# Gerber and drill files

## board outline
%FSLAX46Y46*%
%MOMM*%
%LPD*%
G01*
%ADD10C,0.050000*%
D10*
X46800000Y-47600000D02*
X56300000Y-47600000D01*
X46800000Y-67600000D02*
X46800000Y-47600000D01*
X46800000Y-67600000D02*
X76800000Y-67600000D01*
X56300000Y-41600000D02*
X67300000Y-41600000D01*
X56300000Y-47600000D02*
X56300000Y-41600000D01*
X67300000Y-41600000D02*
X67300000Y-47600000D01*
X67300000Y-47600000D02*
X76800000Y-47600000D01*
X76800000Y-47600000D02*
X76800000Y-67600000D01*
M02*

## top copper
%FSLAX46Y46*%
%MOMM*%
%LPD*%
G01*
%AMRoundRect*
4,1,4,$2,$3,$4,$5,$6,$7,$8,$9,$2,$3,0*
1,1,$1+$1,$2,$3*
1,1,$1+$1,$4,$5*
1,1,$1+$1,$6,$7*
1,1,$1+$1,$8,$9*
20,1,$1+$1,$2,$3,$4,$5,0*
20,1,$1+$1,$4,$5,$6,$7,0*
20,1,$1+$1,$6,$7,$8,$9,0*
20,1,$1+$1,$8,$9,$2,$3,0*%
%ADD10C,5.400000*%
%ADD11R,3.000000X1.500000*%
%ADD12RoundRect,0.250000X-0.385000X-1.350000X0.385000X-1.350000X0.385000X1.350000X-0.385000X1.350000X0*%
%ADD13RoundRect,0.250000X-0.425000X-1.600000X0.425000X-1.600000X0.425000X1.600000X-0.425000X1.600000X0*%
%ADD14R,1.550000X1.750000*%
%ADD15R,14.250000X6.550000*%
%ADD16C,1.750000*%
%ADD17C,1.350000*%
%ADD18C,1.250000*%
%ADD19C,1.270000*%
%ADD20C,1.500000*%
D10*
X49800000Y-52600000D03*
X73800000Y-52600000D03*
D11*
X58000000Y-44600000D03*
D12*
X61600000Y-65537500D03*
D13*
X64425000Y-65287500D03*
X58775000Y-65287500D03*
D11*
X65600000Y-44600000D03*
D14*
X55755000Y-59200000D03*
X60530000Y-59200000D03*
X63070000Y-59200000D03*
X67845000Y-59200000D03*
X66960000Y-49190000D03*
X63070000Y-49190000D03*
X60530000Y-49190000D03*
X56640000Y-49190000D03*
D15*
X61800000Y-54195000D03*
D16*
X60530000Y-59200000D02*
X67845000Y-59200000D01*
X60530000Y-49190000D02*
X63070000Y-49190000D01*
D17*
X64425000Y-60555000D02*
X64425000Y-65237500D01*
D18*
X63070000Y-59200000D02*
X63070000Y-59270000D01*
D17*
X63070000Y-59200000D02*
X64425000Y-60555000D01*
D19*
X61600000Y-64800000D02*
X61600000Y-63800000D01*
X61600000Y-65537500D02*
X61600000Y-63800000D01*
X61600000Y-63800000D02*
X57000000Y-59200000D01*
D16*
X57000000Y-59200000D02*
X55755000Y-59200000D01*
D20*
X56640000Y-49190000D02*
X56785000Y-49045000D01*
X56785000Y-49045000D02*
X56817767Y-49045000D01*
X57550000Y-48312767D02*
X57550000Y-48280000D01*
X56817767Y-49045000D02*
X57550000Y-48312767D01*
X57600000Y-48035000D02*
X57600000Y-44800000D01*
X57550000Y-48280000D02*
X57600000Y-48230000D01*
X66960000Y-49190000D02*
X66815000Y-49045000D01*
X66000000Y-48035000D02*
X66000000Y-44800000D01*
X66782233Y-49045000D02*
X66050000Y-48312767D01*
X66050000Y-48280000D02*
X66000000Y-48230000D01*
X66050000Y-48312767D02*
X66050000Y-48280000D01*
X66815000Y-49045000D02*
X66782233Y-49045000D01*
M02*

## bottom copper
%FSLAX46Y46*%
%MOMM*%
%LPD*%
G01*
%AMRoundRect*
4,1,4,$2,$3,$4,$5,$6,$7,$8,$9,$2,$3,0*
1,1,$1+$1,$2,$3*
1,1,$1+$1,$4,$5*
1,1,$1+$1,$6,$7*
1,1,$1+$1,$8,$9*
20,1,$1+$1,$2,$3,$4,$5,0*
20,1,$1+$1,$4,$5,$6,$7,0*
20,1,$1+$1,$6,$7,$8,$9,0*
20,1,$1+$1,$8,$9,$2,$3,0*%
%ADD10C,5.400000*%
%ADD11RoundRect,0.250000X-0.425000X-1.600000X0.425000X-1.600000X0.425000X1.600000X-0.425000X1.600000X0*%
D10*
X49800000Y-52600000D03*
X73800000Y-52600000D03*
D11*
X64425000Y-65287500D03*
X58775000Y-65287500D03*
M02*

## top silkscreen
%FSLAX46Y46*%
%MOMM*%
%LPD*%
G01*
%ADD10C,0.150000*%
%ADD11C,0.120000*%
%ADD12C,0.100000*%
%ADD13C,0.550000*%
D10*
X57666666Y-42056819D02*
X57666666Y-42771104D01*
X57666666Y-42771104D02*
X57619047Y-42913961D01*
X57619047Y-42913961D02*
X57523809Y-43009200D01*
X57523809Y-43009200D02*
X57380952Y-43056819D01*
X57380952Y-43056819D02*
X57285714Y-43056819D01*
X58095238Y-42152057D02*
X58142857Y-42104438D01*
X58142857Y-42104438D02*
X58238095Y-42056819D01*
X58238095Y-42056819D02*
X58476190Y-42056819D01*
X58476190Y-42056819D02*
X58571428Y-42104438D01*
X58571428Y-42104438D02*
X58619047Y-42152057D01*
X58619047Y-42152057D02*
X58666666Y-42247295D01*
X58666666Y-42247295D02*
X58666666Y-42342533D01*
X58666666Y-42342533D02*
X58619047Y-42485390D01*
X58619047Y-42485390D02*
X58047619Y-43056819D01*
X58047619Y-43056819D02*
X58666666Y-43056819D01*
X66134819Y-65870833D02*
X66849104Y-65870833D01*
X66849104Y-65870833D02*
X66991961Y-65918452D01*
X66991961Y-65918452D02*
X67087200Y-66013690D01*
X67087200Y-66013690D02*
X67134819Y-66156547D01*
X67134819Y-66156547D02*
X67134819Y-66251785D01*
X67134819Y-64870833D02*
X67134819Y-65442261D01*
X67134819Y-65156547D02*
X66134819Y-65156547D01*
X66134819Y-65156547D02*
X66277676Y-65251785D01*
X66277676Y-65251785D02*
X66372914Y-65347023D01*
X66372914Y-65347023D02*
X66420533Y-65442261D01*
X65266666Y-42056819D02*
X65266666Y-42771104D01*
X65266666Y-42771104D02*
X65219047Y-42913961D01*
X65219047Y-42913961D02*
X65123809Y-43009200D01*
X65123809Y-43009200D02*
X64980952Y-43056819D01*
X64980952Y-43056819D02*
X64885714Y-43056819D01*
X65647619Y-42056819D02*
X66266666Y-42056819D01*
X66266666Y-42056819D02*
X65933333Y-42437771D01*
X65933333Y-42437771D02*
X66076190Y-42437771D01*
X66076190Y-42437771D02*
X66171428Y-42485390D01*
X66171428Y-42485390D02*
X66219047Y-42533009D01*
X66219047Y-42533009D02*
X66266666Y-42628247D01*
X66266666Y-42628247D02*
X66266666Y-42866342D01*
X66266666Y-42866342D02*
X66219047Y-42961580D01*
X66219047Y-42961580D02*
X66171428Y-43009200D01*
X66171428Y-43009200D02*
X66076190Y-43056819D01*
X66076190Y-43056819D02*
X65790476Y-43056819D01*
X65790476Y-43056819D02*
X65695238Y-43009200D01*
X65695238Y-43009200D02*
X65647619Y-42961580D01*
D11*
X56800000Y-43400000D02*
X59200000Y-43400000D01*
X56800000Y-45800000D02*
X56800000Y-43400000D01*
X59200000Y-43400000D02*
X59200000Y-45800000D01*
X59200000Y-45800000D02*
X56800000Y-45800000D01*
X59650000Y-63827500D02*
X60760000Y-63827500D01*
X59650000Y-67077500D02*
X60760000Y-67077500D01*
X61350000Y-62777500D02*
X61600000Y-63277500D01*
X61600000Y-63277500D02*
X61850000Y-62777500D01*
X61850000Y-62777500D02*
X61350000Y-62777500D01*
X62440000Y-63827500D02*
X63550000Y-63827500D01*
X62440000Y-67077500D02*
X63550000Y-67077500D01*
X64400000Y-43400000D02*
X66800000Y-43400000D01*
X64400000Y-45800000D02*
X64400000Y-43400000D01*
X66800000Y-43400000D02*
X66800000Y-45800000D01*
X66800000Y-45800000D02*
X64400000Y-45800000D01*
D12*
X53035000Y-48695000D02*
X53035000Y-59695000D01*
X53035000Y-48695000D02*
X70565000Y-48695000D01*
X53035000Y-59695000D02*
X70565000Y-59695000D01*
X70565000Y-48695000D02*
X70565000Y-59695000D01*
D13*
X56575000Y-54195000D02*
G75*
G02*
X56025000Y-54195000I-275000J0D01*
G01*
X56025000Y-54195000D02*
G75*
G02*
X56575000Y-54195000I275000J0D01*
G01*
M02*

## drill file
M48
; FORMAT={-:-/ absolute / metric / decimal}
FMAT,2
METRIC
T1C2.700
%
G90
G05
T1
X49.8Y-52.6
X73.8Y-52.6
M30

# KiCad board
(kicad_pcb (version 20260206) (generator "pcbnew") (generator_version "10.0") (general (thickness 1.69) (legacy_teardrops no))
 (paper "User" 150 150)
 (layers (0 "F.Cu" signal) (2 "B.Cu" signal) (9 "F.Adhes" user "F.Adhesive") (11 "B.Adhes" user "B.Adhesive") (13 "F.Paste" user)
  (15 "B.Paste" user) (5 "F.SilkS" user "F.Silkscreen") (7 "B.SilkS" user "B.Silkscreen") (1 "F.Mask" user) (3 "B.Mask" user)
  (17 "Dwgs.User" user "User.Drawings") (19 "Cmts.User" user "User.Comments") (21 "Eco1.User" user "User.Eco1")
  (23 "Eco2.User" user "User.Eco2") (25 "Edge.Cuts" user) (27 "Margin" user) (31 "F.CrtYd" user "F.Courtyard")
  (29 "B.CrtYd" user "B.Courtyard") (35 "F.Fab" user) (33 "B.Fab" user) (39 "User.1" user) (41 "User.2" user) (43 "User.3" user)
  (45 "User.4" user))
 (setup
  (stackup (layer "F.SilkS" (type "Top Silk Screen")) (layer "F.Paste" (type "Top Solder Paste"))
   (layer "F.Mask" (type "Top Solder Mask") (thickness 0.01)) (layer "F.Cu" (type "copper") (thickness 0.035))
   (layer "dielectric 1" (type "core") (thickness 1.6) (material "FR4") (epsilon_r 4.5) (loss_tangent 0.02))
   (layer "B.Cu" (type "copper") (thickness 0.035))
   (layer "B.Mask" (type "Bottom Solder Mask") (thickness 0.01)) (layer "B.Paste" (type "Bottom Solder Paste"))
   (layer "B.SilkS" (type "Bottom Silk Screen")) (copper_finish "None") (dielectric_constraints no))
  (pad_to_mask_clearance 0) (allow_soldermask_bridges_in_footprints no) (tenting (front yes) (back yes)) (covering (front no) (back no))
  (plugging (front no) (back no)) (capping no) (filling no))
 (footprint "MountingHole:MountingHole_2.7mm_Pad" (layer "F.Cu") (at 49.8 52.6)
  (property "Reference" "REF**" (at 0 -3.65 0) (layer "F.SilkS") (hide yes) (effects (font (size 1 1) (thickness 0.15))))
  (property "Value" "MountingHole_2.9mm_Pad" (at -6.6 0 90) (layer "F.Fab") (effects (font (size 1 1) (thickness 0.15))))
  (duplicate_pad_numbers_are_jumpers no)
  (pad "1" thru_hole circle (at 0 0) (size 5.4 5.4) (drill 2.7) (layers "*.Cu" "*.Mask") (remove_unused_layers no) (zone_connect 2)))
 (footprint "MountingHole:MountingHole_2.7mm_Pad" (layer "F.Cu") (at 73.8 52.6)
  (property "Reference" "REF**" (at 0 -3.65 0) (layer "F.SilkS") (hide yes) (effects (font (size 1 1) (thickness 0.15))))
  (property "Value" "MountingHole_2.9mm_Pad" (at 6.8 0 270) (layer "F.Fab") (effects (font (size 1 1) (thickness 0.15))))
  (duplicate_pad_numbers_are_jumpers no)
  (pad "1" thru_hole circle (at 0 0) (size 5.4 5.4) (drill 2.7) (layers "*.Cu" "*.Mask") (remove_unused_layers no) (zone_connect 2)))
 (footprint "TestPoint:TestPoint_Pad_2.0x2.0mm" (layer "F.Cu") (at 58 44.6)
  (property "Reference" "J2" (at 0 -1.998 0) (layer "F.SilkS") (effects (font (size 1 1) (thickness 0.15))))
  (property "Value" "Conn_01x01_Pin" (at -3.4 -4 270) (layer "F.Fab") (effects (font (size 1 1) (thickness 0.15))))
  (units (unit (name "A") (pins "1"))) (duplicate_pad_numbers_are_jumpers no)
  (fp_line (start -1.2 -1.2) (end 1.2 -1.2) (stroke (width 0.12) (type solid)) (layer "F.SilkS"))
  (fp_line (start -1.2 1.2) (end -1.2 -1.2) (stroke (width 0.12) (type solid)) (layer "F.SilkS"))
  (fp_line (start 1.2 -1.2) (end 1.2 1.2) (stroke (width 0.12) (type solid)) (layer "F.SilkS"))
  (fp_line (start 1.2 1.2) (end -1.2 1.2) (stroke (width 0.12) (type solid)) (layer "F.SilkS"))
  (pad "1" smd rect (at 0 0) (size 3 1.5) (layers "F.Cu" "F.Mask") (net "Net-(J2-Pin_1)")))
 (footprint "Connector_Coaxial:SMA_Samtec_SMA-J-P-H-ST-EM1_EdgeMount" (layer "F.Cu") (at 61.6 65.5375 -90)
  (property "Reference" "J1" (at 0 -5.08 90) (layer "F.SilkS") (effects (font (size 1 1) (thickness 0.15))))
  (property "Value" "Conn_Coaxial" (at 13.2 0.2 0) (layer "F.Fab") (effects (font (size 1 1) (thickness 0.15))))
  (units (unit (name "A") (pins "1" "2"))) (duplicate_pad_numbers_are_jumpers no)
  (fp_line (start -1.71 1.95) (end -1.71 0.84) (stroke (width 0.12) (type solid)) (layer "F.SilkS"))
  (fp_line (start 1.54 1.95) (end 1.54 0.84) (stroke (width 0.12) (type solid)) (layer "F.SilkS"))
  (fp_line (start -2.76 0.25) (end -2.26 0) (stroke (width 0.12) (type solid)) (layer "F.SilkS"))
  (fp_line (start -2.26 0) (end -2.76 -0.25) (stroke (width 0.12) (type solid)) (layer "F.SilkS"))
  (fp_line (start -2.76 -0.25) (end -2.76 0.25) (stroke (width 0.12) (type solid)) (layer "F.SilkS"))
  (fp_line (start -1.71 -0.84) (end -1.71 -1.95) (stroke (width 0.12) (type solid)) (layer "F.SilkS"))
  (fp_line (start 1.54 -0.84) (end 1.54 -1.95) (stroke (width 0.12) (type solid)) (layer "F.SilkS"))
  (pad "1" smd roundrect (at 0 0) (size 1.27 3.2) (layers "F.Cu" "F.Mask") (roundrect_rratio 0.1968503937) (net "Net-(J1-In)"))
  (pad "2" smd roundrect (at -0.25 -2.825) (size 1.35 3.7) (layers "F.Cu" "F.Mask") (roundrect_rratio 0.1851851852) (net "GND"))
  (pad "2" smd roundrect (at -0.25 -2.825) (size 1.35 3.7) (layers "B.Cu" "B.Mask") (roundrect_rratio 0.1851851852) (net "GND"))
  (pad "2" smd roundrect (at -0.25 2.825) (size 1.35 3.7) (layers "F.Cu" "F.Mask") (roundrect_rratio 0.1851851852) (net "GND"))
  (pad "2" smd roundrect (at -0.25 2.825) (size 1.35 3.7) (layers "B.Cu" "B.Mask") (roundrect_rratio 0.1851851852) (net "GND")))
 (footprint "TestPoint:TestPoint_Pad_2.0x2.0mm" (layer "F.Cu") (at 65.6 44.6)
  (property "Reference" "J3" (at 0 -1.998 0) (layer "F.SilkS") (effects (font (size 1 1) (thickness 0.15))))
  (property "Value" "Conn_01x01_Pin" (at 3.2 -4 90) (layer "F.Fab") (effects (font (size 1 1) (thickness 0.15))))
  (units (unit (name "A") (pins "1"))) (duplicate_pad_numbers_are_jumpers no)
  (fp_line (start -1.2 -1.2) (end 1.2 -1.2) (stroke (width 0.12) (type solid)) (layer "F.SilkS"))
  (fp_line (start -1.2 1.2) (end -1.2 -1.2) (stroke (width 0.12) (type solid)) (layer "F.SilkS"))
  (fp_line (start 1.2 -1.2) (end 1.2 1.2) (stroke (width 0.12) (type solid)) (layer "F.SilkS"))
  (fp_line (start 1.2 1.2) (end -1.2 1.2) (stroke (width 0.12) (type solid)) (layer "F.SilkS"))
  (pad "1" smd rect (at 0 0) (size 3 1.5) (layers "F.Cu" "F.Mask") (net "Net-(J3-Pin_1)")))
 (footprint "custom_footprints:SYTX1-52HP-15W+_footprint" (layer "F.Cu") (at 61.8 54.195)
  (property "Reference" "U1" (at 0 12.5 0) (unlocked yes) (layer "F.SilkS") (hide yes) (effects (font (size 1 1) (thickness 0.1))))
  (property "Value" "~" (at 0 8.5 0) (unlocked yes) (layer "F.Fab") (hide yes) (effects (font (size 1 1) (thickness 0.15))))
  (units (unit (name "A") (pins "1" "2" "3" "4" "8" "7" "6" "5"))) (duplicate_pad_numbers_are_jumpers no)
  (fp_line (start -8.765 -5.5) (end -8.765 5.5) (stroke (width 0.1) (type solid)) (layer "F.SilkS"))
  (fp_line (start -8.765 -5.5) (end 8.765 -5.5) (stroke (width 0.1) (type solid)) (layer "F.SilkS"))
  (fp_line (start -8.765 5.5) (end 8.765 5.5) (stroke (width 0.1) (type solid)) (layer "F.SilkS"))
  (fp_line (start 8.765 -5.5) (end 8.765 5.5) (stroke (width 0.1) (type solid)) (layer "F.SilkS"))
  (fp_circle (center -5.5 0) (end -6 0) (stroke (width 0.1) (type solid)) (fill yes) (layer "F.SilkS"))
  (pad "1" smd rect (at -6.045 5.005) (size 1.55 1.75) (layers "F.Cu" "F.Mask" "F.Paste") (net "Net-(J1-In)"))
  (pad "2" smd rect (at -1.27 5.005) (size 1.55 1.75) (layers "F.Cu" "F.Mask" "F.Paste") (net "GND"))
  (pad "3" smd rect (at 1.27 5.005) (size 1.55 1.75) (layers "F.Cu" "F.Mask" "F.Paste") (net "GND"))
  (pad "4" smd rect (at 6.045 5.005) (size 1.55 1.75) (layers "F.Cu" "F.Mask" "F.Paste") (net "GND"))
  (pad "5" smd rect (at 5.16 -5.005) (size 1.55 1.75) (layers "F.Cu" "F.Mask" "F.Paste") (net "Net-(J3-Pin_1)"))
  (pad "6" smd rect (at 1.27 -5.005) (size 1.55 1.75) (layers "F.Cu" "F.Mask" "F.Paste") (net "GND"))
  (pad "7" smd rect (at -1.27 -5.005) (size 1.55 1.75) (layers "F.Cu" "F.Mask" "F.Paste") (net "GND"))
  (pad "8" smd rect (at -5.16 -5.005) (size 1.55 1.75) (layers "F.Cu" "F.Mask" "F.Paste") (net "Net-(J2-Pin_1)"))
  (pad "9" smd rect (at 0 0) (size 14.25 6.55) (layers "F.Cu" "F.Mask" "F.Paste")))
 (gr_line (start 46.8 47.6) (end 56.3 47.6) (stroke (width 0.05) (type solid)) (layer "Edge.Cuts"))
 (gr_line (start 46.8 67.6) (end 46.8 47.6) (stroke (width 0.05) (type solid)) (layer "Edge.Cuts"))
 (gr_line (start 46.8 67.6) (end 76.8 67.6) (stroke (width 0.05) (type solid)) (layer "Edge.Cuts"))
 (gr_line (start 56.3 41.6) (end 67.3 41.6) (stroke (width 0.05) (type solid)) (layer "Edge.Cuts"))
 (gr_line (start 56.3 47.6) (end 56.3 41.6) (stroke (width 0.05) (type solid)) (layer "Edge.Cuts"))
 (gr_line (start 67.3 41.6) (end 67.3 47.6) (stroke (width 0.05) (type solid)) (layer "Edge.Cuts"))
 (gr_line (start 67.3 47.6) (end 76.8 47.6) (stroke (width 0.05) (type solid)) (layer "Edge.Cuts"))
 (gr_line (start 76.8 47.6) (end 76.8 67.6) (stroke (width 0.05) (type solid)) (layer "Edge.Cuts"))
 (segment (start 60.53 59.2) (end 67.845 59.2) (width 1.75) (layer "F.Cu") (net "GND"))
 (segment (start 60.53 49.19) (end 63.07 49.19) (width 1.75) (layer "F.Cu") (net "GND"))
 (segment (start 64.425 60.555) (end 64.425 65.2375) (width 1.35) (layer "F.Cu") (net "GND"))
 (segment (start 63.07 59.2) (end 63.07 59.27) (width 1.25) (layer "F.Cu") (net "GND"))
 (segment (start 63.07 59.2) (end 64.425 60.555) (width 1.35) (layer "F.Cu") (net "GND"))
 (segment (start 61.6 64.8) (end 61.6 63.8) (width 1.27) (layer "F.Cu") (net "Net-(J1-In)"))
 (segment (start 61.6 65.5375) (end 61.6 63.8) (width 1.27) (layer "F.Cu") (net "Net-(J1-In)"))
 (segment (start 61.6 63.8) (end 57 59.2) (width 1.27) (layer "F.Cu") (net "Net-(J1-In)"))
 (segment (start 57 59.2) (end 55.755 59.2) (width 1.75) (layer "F.Cu") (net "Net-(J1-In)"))
 (segment (start 56.64 49.19) (end 56.785 49.045) (width 1.5) (layer "F.Cu") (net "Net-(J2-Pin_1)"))
 (segment (start 56.785 49.045) (end 56.817767 49.045) (width 1.5) (layer "F.Cu") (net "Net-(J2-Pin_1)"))
 (segment (start 57.55 48.312767) (end 57.55 48.28) (width 1.5) (layer "F.Cu") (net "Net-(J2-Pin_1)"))
 (segment (start 56.817767 49.045) (end 57.55 48.312767) (width 1.5) (layer "F.Cu") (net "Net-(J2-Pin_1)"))
 (segment (start 57.6 48.035) (end 57.6 44.8) (width 1.5) (layer "F.Cu") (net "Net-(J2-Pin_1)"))
 (segment (start 57.55 48.28) (end 57.6 48.23) (width 1.5) (layer "F.Cu") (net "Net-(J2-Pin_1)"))
 (segment (start 66.96 49.19) (end 66.815 49.045) (width 1.5) (layer "F.Cu") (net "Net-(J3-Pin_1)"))
 (segment (start 66 48.035) (end 66 44.8) (width 1.5) (layer "F.Cu") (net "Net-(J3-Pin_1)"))
 (segment (start 66.782233 49.045) (end 66.05 48.312767) (width 1.5) (layer "F.Cu") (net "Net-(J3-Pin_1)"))
 (segment (start 66.05 48.28) (end 66 48.23) (width 1.5) (layer "F.Cu") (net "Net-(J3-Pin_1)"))
 (segment (start 66.05 48.312767) (end 66.05 48.28) (width 1.5) (layer "F.Cu") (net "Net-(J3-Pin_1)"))
 (segment (start 66.815 49.045) (end 66.782233 49.045) (width 1.5) (layer "F.Cu") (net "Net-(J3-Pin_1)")))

